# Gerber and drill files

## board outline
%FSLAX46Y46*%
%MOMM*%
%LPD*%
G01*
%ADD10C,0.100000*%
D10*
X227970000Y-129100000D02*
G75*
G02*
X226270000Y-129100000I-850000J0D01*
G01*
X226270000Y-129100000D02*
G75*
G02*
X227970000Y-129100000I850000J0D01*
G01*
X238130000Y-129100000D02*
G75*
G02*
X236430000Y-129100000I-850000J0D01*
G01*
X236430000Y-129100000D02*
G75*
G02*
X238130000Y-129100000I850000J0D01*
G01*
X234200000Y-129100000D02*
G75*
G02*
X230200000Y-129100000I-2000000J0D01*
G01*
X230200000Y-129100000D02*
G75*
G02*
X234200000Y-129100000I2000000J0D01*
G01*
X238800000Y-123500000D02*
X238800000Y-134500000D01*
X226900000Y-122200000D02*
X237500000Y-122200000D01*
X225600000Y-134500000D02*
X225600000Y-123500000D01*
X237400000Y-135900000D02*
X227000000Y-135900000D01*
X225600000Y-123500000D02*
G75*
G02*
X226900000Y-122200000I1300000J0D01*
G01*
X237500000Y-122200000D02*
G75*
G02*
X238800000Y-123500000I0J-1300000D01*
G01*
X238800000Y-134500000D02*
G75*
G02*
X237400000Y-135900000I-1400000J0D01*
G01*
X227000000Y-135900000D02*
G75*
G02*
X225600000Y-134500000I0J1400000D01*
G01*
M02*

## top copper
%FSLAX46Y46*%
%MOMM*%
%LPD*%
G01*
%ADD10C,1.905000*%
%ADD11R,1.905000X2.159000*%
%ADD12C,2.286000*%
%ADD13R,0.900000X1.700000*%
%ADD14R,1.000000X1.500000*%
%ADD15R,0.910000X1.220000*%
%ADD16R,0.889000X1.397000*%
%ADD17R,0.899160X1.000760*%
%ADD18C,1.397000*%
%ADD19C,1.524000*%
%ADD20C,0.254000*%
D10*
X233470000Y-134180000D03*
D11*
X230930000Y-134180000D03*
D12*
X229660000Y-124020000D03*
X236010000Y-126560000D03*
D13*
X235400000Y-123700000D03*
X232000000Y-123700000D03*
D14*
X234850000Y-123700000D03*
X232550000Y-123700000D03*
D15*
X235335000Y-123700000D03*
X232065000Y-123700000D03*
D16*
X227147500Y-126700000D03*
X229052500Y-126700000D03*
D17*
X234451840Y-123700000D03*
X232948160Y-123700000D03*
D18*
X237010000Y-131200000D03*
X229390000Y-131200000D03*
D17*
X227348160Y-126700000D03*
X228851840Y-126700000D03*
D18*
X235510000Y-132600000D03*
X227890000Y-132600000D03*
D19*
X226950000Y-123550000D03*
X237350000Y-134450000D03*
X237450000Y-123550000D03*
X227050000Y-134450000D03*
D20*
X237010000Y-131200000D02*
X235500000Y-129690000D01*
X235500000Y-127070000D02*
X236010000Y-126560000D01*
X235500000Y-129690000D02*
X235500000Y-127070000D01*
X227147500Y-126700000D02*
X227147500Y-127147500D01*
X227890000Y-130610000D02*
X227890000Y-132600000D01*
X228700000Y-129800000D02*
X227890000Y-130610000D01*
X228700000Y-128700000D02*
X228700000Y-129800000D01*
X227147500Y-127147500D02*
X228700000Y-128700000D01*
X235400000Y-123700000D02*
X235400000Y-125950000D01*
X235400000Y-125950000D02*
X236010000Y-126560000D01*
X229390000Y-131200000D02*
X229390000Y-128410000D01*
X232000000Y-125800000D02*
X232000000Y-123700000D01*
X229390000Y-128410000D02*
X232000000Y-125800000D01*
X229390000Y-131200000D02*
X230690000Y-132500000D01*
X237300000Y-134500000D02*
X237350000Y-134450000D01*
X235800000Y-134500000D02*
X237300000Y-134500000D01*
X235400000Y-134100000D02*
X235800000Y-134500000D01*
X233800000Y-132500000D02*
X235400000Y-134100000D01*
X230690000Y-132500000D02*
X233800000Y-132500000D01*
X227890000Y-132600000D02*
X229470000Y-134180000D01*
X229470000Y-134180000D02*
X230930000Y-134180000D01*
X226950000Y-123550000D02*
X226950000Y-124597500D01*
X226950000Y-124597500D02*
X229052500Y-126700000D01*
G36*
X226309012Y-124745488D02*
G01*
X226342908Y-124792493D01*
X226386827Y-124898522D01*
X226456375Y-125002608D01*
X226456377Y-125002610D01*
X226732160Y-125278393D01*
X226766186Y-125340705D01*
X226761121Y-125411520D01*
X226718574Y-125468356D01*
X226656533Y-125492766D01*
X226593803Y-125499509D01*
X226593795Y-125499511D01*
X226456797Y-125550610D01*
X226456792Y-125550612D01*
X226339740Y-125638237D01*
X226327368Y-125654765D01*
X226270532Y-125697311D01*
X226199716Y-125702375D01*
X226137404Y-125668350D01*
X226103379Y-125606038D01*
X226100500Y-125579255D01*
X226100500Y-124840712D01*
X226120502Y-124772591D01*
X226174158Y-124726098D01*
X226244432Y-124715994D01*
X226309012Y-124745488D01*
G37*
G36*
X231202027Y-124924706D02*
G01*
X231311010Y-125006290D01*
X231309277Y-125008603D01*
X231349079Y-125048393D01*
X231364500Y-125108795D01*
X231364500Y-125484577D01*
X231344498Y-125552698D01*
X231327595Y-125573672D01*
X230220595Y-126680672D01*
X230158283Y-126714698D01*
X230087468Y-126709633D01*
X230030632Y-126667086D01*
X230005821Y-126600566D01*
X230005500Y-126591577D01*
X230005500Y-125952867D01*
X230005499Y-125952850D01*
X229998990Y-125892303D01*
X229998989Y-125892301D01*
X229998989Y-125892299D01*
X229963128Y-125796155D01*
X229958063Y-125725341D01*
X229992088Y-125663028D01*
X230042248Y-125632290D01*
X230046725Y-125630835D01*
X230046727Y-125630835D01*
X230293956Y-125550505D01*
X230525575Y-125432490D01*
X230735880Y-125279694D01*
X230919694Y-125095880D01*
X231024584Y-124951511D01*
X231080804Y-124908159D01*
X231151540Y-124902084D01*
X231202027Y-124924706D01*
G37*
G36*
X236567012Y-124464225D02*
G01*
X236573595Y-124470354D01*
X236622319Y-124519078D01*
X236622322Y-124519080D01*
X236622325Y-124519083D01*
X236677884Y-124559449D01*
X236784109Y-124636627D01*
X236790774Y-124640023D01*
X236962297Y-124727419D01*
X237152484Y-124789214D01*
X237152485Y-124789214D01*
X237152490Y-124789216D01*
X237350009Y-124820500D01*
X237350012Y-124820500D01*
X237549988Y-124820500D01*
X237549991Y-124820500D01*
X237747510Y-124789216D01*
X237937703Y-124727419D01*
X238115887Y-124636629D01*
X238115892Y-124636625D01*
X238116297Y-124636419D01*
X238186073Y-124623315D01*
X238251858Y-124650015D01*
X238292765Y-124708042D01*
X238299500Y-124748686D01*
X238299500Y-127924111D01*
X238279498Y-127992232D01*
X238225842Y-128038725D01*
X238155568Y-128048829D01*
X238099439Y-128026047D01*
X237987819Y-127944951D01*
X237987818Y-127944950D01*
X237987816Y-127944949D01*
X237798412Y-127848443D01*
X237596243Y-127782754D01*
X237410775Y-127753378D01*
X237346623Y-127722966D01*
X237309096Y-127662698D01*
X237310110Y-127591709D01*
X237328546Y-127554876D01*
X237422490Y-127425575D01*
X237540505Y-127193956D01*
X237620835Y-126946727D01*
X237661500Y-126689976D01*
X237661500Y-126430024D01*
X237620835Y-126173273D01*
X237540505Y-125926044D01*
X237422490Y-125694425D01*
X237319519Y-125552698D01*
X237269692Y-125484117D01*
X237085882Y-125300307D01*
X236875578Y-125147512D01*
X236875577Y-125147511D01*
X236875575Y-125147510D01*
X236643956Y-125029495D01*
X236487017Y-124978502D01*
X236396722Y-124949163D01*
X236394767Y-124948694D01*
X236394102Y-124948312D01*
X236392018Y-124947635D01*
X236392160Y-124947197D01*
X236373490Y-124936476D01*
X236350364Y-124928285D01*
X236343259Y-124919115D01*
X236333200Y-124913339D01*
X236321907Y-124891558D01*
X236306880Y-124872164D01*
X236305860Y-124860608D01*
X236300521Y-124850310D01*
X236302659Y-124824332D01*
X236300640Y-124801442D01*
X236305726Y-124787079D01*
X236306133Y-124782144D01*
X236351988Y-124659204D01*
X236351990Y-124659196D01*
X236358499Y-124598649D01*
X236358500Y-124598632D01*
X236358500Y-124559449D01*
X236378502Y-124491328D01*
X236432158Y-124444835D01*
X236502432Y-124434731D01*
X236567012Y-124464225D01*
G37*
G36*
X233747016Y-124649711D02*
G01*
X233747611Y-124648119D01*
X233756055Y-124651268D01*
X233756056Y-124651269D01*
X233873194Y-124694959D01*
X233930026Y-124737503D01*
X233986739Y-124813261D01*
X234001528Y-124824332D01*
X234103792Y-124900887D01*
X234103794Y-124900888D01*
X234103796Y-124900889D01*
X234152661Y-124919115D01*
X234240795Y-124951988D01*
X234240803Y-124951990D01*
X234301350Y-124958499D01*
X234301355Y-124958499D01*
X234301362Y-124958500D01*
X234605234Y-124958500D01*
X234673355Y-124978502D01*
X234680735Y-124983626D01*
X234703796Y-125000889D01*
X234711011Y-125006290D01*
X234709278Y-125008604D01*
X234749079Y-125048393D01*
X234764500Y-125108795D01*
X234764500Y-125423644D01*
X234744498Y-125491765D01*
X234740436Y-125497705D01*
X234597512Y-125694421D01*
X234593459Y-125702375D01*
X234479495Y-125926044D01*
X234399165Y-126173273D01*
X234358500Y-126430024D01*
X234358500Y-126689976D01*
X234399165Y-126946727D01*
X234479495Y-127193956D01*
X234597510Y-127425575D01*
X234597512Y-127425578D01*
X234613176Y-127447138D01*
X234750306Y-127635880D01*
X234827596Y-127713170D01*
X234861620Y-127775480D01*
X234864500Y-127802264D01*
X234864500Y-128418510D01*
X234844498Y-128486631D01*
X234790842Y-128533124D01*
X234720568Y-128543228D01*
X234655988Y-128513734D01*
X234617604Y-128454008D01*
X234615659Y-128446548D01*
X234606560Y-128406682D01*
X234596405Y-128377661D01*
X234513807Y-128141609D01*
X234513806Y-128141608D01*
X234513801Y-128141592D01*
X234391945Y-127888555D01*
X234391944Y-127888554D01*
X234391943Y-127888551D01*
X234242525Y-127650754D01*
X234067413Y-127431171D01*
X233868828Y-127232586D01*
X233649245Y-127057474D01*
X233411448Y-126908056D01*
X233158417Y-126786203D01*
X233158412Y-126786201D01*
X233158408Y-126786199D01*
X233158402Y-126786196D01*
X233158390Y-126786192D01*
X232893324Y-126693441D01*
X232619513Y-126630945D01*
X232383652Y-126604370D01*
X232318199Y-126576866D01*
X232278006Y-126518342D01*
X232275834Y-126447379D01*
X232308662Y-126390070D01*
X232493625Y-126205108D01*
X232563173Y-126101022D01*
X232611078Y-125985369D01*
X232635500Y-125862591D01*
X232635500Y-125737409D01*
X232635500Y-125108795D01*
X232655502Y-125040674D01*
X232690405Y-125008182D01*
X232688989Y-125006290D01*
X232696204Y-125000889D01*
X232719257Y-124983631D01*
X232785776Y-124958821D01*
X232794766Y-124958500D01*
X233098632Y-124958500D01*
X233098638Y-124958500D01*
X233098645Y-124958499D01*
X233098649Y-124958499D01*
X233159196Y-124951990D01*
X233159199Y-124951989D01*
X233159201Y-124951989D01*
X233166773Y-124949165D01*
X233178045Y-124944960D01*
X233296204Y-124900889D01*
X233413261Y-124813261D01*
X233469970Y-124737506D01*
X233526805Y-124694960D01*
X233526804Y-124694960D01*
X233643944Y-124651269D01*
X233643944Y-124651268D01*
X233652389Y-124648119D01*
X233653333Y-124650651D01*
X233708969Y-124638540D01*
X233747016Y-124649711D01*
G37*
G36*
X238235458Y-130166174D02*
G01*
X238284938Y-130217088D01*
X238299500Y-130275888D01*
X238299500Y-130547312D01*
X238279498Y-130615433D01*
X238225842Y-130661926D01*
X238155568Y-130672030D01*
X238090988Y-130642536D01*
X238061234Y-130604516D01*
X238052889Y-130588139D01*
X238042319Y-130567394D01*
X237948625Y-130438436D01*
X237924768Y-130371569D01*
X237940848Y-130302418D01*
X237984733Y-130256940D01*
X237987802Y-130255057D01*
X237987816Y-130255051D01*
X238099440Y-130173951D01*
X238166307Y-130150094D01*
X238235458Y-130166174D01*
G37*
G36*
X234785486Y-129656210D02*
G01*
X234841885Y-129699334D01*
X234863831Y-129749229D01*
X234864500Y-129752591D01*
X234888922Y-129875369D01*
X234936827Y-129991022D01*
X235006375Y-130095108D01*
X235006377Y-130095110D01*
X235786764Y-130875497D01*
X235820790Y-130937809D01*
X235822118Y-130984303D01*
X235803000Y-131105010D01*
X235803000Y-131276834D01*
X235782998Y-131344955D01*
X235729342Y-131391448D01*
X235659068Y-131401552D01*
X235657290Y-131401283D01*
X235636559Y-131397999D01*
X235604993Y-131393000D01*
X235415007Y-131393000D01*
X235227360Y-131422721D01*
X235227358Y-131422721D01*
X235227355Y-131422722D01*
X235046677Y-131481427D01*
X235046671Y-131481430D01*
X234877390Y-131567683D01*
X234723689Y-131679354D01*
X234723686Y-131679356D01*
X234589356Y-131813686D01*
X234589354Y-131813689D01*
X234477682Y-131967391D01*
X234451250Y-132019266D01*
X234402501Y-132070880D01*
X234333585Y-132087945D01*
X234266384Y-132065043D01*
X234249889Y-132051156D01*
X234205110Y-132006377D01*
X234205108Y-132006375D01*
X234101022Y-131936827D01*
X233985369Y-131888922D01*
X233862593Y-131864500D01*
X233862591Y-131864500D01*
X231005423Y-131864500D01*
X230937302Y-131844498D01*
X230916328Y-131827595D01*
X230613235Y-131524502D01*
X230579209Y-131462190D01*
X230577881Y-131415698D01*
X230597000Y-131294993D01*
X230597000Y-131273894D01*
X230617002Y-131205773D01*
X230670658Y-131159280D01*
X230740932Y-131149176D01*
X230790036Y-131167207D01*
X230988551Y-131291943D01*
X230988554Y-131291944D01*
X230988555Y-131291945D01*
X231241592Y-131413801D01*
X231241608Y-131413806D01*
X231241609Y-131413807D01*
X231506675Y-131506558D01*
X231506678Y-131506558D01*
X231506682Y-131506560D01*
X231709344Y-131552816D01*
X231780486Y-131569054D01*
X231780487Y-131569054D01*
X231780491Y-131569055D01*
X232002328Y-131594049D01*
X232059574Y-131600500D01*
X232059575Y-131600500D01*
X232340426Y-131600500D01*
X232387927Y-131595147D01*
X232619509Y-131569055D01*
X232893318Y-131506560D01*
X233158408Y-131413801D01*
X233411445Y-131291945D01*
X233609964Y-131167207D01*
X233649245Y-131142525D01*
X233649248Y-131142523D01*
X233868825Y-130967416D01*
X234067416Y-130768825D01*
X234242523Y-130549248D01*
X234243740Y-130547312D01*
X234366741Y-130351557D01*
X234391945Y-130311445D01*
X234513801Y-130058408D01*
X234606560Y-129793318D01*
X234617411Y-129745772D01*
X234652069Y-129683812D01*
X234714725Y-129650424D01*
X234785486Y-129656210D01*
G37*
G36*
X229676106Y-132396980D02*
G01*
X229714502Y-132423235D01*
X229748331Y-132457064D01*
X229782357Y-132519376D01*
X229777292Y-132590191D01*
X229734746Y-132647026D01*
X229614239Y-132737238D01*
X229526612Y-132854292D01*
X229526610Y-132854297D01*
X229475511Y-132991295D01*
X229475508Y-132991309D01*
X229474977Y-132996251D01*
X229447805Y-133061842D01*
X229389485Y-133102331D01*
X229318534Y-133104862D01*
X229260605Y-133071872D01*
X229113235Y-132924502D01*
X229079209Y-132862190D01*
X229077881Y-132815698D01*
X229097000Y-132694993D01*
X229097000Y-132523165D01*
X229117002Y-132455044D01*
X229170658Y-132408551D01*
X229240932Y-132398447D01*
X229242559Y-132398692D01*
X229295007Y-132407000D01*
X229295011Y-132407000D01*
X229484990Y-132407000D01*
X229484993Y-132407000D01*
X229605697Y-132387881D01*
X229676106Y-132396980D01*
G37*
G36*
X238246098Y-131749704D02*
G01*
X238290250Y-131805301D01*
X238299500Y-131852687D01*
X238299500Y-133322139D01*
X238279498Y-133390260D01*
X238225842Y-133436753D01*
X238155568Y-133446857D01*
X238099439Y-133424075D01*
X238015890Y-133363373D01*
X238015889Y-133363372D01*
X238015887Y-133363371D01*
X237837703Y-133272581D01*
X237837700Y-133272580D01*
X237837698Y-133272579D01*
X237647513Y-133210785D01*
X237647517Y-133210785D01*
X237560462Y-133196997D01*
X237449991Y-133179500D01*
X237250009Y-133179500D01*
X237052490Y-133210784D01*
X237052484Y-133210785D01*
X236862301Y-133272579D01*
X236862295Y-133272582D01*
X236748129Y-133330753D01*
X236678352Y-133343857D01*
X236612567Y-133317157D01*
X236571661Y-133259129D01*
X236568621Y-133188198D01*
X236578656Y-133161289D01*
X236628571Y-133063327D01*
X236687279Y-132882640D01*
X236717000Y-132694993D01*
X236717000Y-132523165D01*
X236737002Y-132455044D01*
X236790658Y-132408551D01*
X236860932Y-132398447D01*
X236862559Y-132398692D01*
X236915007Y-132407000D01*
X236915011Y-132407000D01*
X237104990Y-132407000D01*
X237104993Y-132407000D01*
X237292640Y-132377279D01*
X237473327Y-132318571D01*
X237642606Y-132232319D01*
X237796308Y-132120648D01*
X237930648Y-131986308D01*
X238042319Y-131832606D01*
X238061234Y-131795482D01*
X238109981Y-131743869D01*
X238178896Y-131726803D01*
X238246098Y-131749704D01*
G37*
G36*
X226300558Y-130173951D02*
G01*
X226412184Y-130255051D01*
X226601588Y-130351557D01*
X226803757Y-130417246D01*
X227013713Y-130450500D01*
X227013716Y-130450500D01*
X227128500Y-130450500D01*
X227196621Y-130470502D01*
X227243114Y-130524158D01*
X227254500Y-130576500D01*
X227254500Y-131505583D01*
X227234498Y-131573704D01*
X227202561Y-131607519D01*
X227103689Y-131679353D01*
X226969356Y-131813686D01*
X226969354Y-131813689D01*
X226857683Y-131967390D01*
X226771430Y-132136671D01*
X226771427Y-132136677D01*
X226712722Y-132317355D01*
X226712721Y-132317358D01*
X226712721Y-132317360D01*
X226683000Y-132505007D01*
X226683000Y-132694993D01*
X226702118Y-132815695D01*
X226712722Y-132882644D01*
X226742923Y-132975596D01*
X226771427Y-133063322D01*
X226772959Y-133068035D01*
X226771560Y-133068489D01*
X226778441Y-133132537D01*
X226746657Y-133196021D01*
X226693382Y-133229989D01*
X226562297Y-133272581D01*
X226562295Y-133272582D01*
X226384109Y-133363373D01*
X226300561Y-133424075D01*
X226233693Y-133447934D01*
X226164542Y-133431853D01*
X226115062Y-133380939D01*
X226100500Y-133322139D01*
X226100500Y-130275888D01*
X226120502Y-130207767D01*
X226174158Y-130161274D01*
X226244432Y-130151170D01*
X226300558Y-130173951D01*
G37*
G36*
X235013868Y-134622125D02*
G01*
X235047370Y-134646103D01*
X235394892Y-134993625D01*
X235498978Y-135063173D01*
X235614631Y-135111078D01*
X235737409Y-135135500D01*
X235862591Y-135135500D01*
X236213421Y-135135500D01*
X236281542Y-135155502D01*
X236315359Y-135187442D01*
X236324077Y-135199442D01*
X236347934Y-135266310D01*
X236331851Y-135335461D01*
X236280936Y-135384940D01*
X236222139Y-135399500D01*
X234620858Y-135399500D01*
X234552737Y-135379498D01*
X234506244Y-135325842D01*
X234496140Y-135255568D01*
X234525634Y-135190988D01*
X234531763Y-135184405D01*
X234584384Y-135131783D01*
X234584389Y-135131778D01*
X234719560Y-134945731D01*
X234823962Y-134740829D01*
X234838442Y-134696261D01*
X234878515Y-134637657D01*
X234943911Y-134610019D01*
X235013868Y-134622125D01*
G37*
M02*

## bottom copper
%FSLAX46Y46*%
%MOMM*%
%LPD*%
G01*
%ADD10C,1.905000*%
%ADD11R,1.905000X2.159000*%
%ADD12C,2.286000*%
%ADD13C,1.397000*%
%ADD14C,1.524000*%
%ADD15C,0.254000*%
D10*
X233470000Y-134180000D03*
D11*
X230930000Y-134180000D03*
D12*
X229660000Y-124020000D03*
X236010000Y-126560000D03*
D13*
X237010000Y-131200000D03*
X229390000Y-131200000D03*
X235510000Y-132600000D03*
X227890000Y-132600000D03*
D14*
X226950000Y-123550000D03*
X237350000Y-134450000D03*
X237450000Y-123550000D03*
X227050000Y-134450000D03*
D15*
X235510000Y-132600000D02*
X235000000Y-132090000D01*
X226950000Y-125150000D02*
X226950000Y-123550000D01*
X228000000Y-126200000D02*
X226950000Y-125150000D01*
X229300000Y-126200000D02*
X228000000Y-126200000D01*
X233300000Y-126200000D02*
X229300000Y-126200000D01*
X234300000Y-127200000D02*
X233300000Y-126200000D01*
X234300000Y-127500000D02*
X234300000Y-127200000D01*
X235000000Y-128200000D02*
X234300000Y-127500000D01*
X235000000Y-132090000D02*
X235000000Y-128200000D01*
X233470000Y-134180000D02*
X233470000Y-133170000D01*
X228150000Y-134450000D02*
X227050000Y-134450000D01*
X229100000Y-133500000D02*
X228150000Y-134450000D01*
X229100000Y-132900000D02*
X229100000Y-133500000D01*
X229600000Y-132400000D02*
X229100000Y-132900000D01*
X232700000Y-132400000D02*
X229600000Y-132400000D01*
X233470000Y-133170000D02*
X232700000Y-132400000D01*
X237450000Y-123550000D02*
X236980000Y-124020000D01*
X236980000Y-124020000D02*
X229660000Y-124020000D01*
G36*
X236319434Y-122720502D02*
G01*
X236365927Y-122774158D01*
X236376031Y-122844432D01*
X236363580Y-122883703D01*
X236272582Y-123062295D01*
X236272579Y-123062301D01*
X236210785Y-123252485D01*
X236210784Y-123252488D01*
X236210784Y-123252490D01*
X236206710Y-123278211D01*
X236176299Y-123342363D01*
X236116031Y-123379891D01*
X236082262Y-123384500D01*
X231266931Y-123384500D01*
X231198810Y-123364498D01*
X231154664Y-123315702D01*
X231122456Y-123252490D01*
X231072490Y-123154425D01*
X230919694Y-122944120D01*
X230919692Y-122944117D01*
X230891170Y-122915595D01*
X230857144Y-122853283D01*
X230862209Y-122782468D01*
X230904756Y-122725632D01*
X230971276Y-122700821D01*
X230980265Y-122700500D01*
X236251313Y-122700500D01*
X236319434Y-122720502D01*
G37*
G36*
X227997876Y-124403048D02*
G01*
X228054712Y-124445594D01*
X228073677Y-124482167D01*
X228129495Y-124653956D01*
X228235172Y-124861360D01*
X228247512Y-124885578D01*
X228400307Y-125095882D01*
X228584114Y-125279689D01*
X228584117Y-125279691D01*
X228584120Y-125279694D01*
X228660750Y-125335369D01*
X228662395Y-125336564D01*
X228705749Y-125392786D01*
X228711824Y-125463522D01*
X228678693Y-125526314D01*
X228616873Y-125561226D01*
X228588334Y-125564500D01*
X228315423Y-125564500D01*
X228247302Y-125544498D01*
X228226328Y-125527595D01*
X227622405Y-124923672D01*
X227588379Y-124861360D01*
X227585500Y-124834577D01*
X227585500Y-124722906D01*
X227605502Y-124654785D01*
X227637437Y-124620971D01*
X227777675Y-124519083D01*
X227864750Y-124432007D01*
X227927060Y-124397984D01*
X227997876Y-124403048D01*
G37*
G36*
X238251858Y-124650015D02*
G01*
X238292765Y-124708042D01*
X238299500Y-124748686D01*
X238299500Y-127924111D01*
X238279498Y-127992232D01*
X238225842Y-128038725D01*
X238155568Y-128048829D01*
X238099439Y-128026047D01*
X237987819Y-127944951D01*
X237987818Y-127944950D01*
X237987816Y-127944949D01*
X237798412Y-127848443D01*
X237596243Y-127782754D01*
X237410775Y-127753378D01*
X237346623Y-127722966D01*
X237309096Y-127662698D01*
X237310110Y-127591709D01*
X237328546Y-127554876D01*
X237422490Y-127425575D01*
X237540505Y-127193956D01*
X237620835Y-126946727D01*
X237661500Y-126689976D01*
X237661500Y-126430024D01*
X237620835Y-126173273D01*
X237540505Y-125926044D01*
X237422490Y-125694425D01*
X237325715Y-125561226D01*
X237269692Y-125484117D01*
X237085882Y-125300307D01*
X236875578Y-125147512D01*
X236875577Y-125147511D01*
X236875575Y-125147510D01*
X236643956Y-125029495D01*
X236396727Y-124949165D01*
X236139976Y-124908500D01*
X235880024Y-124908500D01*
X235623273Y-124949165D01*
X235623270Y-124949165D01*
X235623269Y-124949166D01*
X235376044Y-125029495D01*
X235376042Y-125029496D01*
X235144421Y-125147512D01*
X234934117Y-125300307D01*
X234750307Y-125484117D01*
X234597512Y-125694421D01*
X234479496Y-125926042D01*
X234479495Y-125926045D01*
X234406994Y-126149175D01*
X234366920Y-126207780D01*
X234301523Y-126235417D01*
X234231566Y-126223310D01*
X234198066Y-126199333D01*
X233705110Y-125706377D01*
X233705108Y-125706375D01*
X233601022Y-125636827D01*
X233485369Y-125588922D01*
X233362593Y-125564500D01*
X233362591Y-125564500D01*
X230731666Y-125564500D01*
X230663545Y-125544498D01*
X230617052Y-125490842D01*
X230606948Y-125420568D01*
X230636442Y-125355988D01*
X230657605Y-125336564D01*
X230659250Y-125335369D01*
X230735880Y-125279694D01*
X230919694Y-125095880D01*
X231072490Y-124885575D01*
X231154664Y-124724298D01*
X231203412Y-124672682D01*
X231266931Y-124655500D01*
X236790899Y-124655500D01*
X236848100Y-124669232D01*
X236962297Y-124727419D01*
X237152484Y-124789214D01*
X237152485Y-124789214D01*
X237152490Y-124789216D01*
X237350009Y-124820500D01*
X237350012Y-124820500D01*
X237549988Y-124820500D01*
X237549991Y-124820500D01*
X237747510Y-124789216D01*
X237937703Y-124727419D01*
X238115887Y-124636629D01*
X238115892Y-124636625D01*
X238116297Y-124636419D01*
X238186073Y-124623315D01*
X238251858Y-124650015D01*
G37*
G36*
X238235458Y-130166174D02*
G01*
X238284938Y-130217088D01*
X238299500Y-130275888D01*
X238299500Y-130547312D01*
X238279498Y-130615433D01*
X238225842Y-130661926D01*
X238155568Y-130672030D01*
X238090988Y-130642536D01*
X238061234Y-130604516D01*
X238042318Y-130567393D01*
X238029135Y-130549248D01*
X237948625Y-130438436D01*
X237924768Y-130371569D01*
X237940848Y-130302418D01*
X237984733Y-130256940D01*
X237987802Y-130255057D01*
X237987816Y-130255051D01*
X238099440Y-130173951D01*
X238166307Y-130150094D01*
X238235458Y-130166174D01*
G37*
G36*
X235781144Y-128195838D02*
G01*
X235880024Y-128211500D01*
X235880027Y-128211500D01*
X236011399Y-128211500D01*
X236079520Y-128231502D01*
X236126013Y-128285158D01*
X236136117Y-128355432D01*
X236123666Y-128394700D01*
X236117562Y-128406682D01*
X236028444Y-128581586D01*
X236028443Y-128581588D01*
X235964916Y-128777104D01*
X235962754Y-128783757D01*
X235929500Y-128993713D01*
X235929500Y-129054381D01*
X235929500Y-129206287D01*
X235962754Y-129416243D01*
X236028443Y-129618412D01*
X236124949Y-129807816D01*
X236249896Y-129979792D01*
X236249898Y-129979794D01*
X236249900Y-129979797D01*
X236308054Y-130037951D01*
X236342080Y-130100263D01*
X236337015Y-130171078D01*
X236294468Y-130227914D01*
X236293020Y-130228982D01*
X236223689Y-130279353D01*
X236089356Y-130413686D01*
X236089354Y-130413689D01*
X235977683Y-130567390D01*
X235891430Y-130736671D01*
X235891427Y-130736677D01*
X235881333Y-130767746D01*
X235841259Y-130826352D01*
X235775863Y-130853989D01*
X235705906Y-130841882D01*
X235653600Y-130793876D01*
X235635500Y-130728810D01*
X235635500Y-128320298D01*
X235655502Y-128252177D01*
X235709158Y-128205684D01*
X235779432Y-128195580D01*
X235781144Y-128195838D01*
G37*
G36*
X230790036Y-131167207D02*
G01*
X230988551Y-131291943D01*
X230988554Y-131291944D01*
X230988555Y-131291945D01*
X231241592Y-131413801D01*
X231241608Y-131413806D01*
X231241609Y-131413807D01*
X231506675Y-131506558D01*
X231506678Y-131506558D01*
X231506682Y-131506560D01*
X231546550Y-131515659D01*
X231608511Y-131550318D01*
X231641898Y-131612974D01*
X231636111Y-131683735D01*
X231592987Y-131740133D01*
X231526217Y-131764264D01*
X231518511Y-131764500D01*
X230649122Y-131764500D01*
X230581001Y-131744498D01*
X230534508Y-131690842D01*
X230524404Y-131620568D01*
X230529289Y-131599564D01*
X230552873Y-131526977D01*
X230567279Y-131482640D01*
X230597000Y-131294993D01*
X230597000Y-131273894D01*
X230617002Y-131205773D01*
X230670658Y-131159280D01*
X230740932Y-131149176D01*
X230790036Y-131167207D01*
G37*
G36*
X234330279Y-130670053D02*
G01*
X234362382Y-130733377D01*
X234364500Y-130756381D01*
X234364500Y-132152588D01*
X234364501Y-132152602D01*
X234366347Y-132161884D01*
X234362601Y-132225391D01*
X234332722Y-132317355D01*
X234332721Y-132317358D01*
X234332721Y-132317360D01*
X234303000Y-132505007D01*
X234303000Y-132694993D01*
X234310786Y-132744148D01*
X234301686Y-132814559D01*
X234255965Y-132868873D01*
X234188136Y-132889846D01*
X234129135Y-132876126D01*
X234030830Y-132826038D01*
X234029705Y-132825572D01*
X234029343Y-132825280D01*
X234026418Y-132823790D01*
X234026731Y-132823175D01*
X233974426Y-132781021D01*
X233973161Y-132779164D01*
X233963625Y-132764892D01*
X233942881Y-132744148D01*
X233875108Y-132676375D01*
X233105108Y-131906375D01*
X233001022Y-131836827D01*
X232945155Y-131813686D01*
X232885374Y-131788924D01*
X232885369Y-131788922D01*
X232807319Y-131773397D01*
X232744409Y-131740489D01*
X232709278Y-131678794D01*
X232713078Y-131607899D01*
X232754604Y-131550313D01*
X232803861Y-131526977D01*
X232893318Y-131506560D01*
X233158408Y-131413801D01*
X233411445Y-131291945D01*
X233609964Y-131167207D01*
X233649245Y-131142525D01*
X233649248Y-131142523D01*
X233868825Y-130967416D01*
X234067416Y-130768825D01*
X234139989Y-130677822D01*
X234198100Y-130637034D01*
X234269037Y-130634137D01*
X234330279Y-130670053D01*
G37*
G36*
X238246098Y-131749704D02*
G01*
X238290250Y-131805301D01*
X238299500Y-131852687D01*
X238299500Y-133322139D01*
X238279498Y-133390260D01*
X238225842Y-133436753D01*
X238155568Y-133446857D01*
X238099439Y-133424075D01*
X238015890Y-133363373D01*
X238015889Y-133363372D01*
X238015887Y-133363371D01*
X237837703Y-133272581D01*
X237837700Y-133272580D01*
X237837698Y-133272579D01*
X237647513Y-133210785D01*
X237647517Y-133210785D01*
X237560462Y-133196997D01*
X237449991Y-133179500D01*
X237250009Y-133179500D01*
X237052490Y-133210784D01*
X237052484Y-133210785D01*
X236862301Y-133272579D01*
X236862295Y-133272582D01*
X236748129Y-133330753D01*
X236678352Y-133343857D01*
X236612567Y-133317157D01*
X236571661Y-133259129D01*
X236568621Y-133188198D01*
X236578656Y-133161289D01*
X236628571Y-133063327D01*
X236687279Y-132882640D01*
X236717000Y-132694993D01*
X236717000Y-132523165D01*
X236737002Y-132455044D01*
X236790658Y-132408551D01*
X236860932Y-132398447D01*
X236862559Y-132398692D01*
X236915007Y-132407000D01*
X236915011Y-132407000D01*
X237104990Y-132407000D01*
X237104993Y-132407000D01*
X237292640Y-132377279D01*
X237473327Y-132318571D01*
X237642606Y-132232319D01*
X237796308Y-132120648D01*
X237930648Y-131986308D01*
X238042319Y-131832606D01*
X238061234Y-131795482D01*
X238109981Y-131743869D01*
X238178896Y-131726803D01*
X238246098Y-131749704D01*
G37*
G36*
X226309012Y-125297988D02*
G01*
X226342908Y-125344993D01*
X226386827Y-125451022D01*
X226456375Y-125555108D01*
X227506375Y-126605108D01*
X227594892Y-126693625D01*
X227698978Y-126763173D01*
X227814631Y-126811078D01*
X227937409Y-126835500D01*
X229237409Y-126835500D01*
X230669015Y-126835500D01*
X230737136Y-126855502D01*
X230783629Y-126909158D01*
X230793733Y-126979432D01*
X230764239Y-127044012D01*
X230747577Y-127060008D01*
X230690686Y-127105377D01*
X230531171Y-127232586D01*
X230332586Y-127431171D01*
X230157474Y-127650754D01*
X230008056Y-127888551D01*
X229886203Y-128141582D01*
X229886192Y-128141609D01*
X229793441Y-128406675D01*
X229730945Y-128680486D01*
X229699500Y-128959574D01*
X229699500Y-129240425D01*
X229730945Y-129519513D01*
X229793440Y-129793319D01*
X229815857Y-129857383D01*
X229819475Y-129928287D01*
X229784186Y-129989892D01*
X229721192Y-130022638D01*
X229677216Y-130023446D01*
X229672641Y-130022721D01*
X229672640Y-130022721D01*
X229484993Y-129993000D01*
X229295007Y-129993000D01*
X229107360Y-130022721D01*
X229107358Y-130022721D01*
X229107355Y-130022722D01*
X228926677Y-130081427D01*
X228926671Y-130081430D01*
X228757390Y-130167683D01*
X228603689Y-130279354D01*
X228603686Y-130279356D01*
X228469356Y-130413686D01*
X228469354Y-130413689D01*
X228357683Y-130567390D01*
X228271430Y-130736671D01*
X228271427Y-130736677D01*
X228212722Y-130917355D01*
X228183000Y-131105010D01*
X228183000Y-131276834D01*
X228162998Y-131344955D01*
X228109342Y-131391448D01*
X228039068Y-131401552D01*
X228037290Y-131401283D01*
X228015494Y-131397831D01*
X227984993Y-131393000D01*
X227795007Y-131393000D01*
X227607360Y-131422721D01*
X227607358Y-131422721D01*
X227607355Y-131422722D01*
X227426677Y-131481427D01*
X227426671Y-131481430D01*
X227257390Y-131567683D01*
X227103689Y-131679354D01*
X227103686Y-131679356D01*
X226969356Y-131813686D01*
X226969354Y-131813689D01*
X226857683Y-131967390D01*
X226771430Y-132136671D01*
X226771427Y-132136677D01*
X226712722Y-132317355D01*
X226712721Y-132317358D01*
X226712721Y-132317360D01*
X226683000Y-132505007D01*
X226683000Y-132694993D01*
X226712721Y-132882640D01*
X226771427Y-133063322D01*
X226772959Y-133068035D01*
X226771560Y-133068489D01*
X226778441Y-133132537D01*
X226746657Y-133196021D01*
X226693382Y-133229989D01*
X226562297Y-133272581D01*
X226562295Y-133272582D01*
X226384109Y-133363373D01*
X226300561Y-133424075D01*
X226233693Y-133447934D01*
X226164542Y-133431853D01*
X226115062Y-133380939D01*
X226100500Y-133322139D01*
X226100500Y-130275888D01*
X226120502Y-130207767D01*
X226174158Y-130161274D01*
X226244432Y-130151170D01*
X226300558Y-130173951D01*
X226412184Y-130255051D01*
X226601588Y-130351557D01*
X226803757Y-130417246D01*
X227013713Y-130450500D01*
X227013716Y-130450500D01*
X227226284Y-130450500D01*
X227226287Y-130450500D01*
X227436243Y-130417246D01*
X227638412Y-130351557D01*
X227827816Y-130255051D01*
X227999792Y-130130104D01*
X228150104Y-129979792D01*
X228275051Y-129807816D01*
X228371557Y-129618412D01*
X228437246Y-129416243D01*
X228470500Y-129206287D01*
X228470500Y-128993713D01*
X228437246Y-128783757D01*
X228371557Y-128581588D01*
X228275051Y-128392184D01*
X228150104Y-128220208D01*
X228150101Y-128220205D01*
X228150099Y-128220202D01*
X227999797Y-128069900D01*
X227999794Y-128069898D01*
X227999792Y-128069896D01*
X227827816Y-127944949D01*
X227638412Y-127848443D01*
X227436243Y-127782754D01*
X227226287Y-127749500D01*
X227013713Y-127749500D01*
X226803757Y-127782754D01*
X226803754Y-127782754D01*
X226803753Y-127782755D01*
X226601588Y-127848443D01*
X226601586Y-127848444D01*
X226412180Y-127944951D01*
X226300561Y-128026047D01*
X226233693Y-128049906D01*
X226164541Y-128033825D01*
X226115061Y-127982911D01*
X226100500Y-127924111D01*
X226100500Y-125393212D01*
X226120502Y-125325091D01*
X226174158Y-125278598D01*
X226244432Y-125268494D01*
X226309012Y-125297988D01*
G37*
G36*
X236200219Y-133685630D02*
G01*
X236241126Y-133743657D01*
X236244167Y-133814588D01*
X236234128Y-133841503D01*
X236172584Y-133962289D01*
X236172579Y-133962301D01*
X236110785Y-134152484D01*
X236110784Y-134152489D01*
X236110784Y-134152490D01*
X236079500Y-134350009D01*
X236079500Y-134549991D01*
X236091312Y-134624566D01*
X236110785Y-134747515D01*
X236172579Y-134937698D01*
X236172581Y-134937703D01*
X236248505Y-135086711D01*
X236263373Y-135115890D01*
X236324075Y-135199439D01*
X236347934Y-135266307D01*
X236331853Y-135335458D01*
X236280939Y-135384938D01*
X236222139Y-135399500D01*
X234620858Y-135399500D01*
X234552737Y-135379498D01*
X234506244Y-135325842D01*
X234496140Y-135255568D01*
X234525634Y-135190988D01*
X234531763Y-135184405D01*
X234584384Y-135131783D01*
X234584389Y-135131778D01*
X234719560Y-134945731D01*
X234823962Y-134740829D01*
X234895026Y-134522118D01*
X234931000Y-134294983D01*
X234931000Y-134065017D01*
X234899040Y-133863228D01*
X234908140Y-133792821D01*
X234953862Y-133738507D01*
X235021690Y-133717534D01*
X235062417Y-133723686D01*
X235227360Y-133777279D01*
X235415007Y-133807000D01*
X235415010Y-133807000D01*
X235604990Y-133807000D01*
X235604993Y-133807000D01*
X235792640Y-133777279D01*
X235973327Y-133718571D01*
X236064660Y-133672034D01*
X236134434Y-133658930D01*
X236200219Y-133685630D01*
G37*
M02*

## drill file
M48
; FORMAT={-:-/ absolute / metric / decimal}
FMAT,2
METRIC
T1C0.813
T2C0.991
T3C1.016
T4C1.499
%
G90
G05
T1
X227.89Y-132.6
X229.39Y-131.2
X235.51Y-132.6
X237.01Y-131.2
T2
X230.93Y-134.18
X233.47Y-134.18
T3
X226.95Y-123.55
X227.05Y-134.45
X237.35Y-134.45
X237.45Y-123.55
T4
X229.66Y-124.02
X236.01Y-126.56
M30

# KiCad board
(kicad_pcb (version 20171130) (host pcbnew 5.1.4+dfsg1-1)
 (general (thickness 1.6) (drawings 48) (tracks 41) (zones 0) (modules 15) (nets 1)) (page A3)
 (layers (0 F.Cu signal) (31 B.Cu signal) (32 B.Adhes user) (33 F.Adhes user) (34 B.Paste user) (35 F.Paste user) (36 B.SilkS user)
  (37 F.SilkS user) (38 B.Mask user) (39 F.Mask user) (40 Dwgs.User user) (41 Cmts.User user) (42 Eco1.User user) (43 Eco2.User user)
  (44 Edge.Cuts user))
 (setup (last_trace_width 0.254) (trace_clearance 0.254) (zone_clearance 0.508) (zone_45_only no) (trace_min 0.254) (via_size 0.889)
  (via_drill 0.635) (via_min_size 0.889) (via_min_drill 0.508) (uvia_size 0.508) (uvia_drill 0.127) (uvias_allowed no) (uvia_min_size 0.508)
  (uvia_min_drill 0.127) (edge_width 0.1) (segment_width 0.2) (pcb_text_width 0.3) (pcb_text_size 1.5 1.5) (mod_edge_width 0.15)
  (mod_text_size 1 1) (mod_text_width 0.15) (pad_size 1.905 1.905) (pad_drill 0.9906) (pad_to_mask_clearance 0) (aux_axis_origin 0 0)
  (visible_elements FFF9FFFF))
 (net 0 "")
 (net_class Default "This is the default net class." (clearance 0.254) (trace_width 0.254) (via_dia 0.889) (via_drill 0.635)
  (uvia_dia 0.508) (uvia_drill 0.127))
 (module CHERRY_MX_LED (layer F.Cu) (at 232.2 129.1)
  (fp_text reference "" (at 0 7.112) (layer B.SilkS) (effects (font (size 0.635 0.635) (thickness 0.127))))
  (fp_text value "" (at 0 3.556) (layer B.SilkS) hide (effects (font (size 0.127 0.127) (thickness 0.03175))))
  (pad C thru_hole circle (at 1.27 5.08) (size 1.905 1.905) (drill 0.9906) (layers *.Cu *.SilkS *.Mask))
  (pad A thru_hole rect (at -1.27 5.08) (size 1.905 2.159) (drill 0.9906) (layers *.Cu *.SilkS *.Mask)))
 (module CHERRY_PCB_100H (layer F.Cu) (at 232.2 129.1)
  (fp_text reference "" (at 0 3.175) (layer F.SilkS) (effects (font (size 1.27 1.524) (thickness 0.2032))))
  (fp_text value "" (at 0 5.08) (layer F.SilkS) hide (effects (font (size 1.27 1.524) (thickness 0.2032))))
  (pad 1 thru_hole circle (at -2.54 -5.08) (size 2.286 2.286) (drill 1.4986) (layers *.Cu *.SilkS *.Mask))
  (pad 2 thru_hole circle (at 3.81 -2.54) (size 2.286 2.286) (drill 1.4986) (layers *.Cu *.SilkS *.Mask)))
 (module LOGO (layer F.Cu) (at 231.4 125.9)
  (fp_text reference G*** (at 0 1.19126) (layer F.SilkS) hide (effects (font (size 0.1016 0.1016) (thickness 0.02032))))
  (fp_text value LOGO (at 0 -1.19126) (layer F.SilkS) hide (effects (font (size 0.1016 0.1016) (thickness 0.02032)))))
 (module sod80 (layer F.Cu) (at 233.7 123.7)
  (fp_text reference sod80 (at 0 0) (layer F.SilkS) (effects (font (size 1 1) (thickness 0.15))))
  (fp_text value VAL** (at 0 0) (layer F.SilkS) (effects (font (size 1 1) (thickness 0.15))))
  (pad 5 smd rect (at 1.7 0) (size 0.9 1.7) (layers F.Cu F.Paste F.Mask))
  (pad 6 smd rect (at -1.7 0) (size 0.9 1.7) (layers F.Cu F.Paste F.Mask)))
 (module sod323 (layer F.Cu) (at 233.7 123.7)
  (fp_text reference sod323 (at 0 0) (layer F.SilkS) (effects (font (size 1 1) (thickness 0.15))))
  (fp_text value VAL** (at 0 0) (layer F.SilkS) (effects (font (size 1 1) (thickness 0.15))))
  (pad 3 smd rect (at 1.15 0) (size 1 1.5) (layers F.Cu F.Paste F.Mask))
  (pad 4 smd rect (at -1.15 0) (size 1 1.5) (layers F.Cu F.Paste F.Mask)))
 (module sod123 (layer F.Cu) (at 233.7 123.7)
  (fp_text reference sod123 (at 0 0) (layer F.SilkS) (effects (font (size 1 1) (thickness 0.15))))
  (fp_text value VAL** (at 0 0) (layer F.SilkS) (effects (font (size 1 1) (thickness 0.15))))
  (pad 1 smd rect (at 1.635 0) (size 0.91 1.22) (layers F.Cu F.Paste F.Mask))
  (pad 2 smd rect (at -1.635 0) (size 0.91 1.22) (layers F.Cu F.Paste F.Mask)))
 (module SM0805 (layer F.Cu) (at 228.1 126.7)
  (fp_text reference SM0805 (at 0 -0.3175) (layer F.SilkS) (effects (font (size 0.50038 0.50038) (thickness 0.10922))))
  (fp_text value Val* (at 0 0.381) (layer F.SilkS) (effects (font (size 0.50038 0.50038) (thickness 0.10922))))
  (pad 1 smd rect (at -0.9525 0) (size 0.889 1.397) (layers F.Cu F.Paste F.Mask))
  (pad 2 smd rect (at 0.9525 0) (size 0.889 1.397) (layers F.Cu F.Paste F.Mask)))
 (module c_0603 (layer F.Cu) (at 233.7 123.7)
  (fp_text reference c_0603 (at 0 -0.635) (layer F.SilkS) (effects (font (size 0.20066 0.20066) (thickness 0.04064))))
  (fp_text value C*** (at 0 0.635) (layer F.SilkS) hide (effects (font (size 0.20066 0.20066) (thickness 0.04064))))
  (pad 1 smd rect (at 0.75184 0) (size 0.89916 1.00076) (layers F.Cu F.Paste F.Mask))
  (pad 2 smd rect (at -0.75184 0) (size 0.89916 1.00076) (layers F.Cu F.Paste F.Mask)))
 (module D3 (layer F.Cu) (at 233.2 131.2)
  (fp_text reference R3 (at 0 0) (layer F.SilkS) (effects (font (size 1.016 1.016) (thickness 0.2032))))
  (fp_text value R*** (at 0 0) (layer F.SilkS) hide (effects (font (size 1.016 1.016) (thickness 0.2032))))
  (pad 2 thru_hole circle (at 3.81 0) (size 1.397 1.397) (drill 0.8128) (layers *.Cu *.Mask F.SilkS))
  (pad 1 thru_hole circle (at -3.81 0) (size 1.397 1.397) (drill 0.8128) (layers *.Cu *.Mask F.SilkS)))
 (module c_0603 (layer F.Cu) (at 228.1 126.7 180)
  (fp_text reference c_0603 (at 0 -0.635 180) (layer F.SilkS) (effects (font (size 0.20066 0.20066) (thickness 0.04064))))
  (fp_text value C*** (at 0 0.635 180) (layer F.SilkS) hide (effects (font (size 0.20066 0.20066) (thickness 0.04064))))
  (pad 1 smd rect (at 0.75184 0 180) (size 0.89916 1.00076) (layers F.Cu F.Paste F.Mask))
  (pad 2 smd rect (at -0.75184 0 180) (size 0.89916 1.00076) (layers F.Cu F.Paste F.Mask)))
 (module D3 (layer F.Cu) (at 231.7 132.6)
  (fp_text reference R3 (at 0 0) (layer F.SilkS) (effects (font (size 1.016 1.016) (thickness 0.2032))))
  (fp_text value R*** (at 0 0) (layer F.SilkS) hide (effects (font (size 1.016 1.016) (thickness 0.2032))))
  (pad 2 thru_hole circle (at 3.81 0) (size 1.397 1.397) (drill 0.8128) (layers *.Cu *.Mask F.SilkS))
  (pad 1 thru_hole circle (at -3.81 0) (size 1.397 1.397) (drill 0.8128) (layers *.Cu *.Mask F.SilkS)))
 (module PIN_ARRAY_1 (layer F.Cu) (at 226.95 123.55)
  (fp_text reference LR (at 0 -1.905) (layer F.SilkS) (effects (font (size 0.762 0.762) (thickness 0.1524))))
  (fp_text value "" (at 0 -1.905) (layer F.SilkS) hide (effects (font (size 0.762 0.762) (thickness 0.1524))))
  (pad 1 thru_hole circle (at 0 0) (size 1.524 1.524) (drill 1.016) (layers *.Cu *.Mask F.SilkS)))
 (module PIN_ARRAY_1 (layer F.Cu) (at 237.35 134.45)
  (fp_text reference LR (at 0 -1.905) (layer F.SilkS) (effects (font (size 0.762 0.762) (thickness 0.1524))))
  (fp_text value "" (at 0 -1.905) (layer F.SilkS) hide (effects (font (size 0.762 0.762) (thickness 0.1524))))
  (pad 1 thru_hole circle (at 0 0) (size 1.524 1.524) (drill 1.016) (layers *.Cu *.Mask F.SilkS)))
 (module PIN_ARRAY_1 (layer F.Cu) (at 237.45 123.55)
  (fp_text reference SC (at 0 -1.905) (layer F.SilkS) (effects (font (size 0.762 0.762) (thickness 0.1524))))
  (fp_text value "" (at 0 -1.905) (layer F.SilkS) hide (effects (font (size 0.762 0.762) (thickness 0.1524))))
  (pad 1 thru_hole circle (at 0 0) (size 1.524 1.524) (drill 1.016) (layers *.Cu *.Mask F.SilkS)))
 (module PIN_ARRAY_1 (layer F.Cu) (at 227.05 134.45)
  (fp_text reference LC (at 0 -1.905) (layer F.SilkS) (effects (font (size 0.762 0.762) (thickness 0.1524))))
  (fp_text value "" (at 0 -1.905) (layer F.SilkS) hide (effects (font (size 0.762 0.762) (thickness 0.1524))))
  (pad 1 thru_hole circle (at 0 0) (size 1.524 1.524) (drill 1.016) (layers *.Cu *.Mask F.SilkS)))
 (gr_circle (center 227.12 129.1) (end 227.12 128.25) (layer Edge.Cuts) (width 0.1))
 (gr_circle (center 237.28 129.1) (end 237.28 128.25) (layer Edge.Cuts) (width 0.1))
 (gr_circle (center 232.2 129.1) (end 232.2 127.1) (layer Edge.Cuts) (width 0.1))
 (gr_line (start 238.8 123.5) (end 238.8 134.5) (angle 90) (layer Edge.Cuts) (width 0.1))
 (gr_line (start 226.9 122.2) (end 237.5 122.2) (angle 90) (layer Edge.Cuts) (width 0.1))
 (gr_line (start 225.6 134.5) (end 225.6 123.5) (angle 90) (layer Edge.Cuts) (width 0.1))
 (gr_line (start 237.4 135.9) (end 227 135.9) (angle 90) (layer Edge.Cuts) (width 0.1))
 (gr_arc (start 226.9 123.5) (end 225.6 123.5) (angle 90) (layer Edge.Cuts) (width 0.1))
 (gr_arc (start 237.5 123.5) (end 237.5 122.2) (angle 90) (layer Edge.Cuts) (width 0.1))
 (gr_arc (start 237.4 134.5) (end 238.8 134.5) (angle 90) (layer Edge.Cuts) (width 0.1))
 (gr_arc (start 227 134.5) (end 227 135.9) (angle 90) (layer Edge.Cuts) (width 0.1))
 (segment (start 237.01 131.2) (end 235.5 129.69) (width 0.254) (layer F.Cu) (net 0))
 (segment (start 235.5 127.07) (end 236.01 126.56) (width 0.254) (layer F.Cu) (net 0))
 (segment (start 235.5 129.69) (end 235.5 127.07) (width 0.254) (layer F.Cu) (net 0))
 (segment (start 235.51 132.6) (end 235 132.09) (width 0.254) (layer B.Cu) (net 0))
 (segment (start 226.95 125.15) (end 226.95 123.55) (width 0.254) (layer B.Cu) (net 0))
 (segment (start 228 126.2) (end 226.95 125.15) (width 0.254) (layer B.Cu) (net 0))
 (segment (start 229.3 126.2) (end 228 126.2) (width 0.254) (layer B.Cu) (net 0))
 (segment (start 233.3 126.2) (end 229.3 126.2) (width 0.254) (layer B.Cu) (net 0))
 (segment (start 234.3 127.2) (end 233.3 126.2) (width 0.254) (layer B.Cu) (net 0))
 (segment (start 234.3 127.5) (end 234.3 127.2) (width 0.254) (layer B.Cu) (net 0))
 (segment (start 235 128.2) (end 234.3 127.5) (width 0.254) (layer B.Cu) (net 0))
 (segment (start 235 132.09) (end 235 128.2) (width 0.254) (layer B.Cu) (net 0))
 (segment (start 233.47 134.18) (end 233.47 133.17) (width 0.254) (layer B.Cu) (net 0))
 (segment (start 228.15 134.45) (end 227.05 134.45) (width 0.254) (layer B.Cu) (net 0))
 (segment (start 229.1 133.5) (end 228.15 134.45) (width 0.254) (layer B.Cu) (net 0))
 (segment (start 229.1 132.9) (end 229.1 133.5) (width 0.254) (layer B.Cu) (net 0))
 (segment (start 229.6 132.4) (end 229.1 132.9) (width 0.254) (layer B.Cu) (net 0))
 (segment (start 232.7 132.4) (end 229.6 132.4) (width 0.254) (layer B.Cu) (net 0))
 (segment (start 233.47 133.17) (end 232.7 132.4) (width 0.254) (layer B.Cu) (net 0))
 (segment (start 227.1475 126.7) (end 227.1475 127.1475) (width 0.254) (layer F.Cu) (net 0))
 (segment (start 227.89 130.61) (end 227.89 132.6) (width 0.254) (layer F.Cu) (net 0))
 (segment (start 228.7 129.8) (end 227.89 130.61) (width 0.254) (layer F.Cu) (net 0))
 (segment (start 228.7 128.7) (end 228.7 129.8) (width 0.254) (layer F.Cu) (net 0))
 (segment (start 227.1475 127.1475) (end 228.7 128.7) (width 0.254) (layer F.Cu) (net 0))
 (segment (start 237.45 123.55) (end 236.98 124.02) (width 0.254) (layer B.Cu) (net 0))
 (segment (start 236.98 124.02) (end 229.66 124.02) (width 0.254) (layer B.Cu) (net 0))
 (segment (start 235.4 123.7) (end 235.4 125.95) (width 0.254) (layer F.Cu) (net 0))
 (segment (start 235.4 125.95) (end 236.01 126.56) (width 0.254) (layer F.Cu) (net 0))
 (segment (start 229.39 131.2) (end 229.39 128.41) (width 0.254) (layer F.Cu) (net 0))
 (segment (start 232 125.8) (end 232 123.7) (width 0.254) (layer F.Cu) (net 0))
 (segment (start 229.39 128.41) (end 232 125.8) (width 0.254) (layer F.Cu) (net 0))
 (segment (start 229.39 131.2) (end 230.69 132.5) (width 0.254) (layer F.Cu) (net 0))
 (segment (start 237.3 134.5) (end 237.35 134.45) (width 0.254) (layer F.Cu) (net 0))
 (segment (start 235.8 134.5) (end 237.3 134.5) (width 0.254) (layer F.Cu) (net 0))
 (segment (start 235.4 134.1) (end 235.8 134.5) (width 0.254) (layer F.Cu) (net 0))
 (segment (start 233.8 132.5) (end 235.4 134.1) (width 0.254) (layer F.Cu) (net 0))
 (segment (start 230.69 132.5) (end 233.8 132.5) (width 0.254) (layer F.Cu) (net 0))
 (segment (start 227.89 132.6) (end 229.47 134.18) (width 0.254) (layer F.Cu) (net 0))
 (segment (start 229.47 134.18) (end 230.93 134.18) (width 0.254) (layer F.Cu) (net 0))
 (segment (start 226.95 123.55) (end 226.95 124.5975) (width 0.254) (layer F.Cu) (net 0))
 (segment (start 226.95 124.5975) (end 229.0525 126.7) (width 0.254) (layer F.Cu) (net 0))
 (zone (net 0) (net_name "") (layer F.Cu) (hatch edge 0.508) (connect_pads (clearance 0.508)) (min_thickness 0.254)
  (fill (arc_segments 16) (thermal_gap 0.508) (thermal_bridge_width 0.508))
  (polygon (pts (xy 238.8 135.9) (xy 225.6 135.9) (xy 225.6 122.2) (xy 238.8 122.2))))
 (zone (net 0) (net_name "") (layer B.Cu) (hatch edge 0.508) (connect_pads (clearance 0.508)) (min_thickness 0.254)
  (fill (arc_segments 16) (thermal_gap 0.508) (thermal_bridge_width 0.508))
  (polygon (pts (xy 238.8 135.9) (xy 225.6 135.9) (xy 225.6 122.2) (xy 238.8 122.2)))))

